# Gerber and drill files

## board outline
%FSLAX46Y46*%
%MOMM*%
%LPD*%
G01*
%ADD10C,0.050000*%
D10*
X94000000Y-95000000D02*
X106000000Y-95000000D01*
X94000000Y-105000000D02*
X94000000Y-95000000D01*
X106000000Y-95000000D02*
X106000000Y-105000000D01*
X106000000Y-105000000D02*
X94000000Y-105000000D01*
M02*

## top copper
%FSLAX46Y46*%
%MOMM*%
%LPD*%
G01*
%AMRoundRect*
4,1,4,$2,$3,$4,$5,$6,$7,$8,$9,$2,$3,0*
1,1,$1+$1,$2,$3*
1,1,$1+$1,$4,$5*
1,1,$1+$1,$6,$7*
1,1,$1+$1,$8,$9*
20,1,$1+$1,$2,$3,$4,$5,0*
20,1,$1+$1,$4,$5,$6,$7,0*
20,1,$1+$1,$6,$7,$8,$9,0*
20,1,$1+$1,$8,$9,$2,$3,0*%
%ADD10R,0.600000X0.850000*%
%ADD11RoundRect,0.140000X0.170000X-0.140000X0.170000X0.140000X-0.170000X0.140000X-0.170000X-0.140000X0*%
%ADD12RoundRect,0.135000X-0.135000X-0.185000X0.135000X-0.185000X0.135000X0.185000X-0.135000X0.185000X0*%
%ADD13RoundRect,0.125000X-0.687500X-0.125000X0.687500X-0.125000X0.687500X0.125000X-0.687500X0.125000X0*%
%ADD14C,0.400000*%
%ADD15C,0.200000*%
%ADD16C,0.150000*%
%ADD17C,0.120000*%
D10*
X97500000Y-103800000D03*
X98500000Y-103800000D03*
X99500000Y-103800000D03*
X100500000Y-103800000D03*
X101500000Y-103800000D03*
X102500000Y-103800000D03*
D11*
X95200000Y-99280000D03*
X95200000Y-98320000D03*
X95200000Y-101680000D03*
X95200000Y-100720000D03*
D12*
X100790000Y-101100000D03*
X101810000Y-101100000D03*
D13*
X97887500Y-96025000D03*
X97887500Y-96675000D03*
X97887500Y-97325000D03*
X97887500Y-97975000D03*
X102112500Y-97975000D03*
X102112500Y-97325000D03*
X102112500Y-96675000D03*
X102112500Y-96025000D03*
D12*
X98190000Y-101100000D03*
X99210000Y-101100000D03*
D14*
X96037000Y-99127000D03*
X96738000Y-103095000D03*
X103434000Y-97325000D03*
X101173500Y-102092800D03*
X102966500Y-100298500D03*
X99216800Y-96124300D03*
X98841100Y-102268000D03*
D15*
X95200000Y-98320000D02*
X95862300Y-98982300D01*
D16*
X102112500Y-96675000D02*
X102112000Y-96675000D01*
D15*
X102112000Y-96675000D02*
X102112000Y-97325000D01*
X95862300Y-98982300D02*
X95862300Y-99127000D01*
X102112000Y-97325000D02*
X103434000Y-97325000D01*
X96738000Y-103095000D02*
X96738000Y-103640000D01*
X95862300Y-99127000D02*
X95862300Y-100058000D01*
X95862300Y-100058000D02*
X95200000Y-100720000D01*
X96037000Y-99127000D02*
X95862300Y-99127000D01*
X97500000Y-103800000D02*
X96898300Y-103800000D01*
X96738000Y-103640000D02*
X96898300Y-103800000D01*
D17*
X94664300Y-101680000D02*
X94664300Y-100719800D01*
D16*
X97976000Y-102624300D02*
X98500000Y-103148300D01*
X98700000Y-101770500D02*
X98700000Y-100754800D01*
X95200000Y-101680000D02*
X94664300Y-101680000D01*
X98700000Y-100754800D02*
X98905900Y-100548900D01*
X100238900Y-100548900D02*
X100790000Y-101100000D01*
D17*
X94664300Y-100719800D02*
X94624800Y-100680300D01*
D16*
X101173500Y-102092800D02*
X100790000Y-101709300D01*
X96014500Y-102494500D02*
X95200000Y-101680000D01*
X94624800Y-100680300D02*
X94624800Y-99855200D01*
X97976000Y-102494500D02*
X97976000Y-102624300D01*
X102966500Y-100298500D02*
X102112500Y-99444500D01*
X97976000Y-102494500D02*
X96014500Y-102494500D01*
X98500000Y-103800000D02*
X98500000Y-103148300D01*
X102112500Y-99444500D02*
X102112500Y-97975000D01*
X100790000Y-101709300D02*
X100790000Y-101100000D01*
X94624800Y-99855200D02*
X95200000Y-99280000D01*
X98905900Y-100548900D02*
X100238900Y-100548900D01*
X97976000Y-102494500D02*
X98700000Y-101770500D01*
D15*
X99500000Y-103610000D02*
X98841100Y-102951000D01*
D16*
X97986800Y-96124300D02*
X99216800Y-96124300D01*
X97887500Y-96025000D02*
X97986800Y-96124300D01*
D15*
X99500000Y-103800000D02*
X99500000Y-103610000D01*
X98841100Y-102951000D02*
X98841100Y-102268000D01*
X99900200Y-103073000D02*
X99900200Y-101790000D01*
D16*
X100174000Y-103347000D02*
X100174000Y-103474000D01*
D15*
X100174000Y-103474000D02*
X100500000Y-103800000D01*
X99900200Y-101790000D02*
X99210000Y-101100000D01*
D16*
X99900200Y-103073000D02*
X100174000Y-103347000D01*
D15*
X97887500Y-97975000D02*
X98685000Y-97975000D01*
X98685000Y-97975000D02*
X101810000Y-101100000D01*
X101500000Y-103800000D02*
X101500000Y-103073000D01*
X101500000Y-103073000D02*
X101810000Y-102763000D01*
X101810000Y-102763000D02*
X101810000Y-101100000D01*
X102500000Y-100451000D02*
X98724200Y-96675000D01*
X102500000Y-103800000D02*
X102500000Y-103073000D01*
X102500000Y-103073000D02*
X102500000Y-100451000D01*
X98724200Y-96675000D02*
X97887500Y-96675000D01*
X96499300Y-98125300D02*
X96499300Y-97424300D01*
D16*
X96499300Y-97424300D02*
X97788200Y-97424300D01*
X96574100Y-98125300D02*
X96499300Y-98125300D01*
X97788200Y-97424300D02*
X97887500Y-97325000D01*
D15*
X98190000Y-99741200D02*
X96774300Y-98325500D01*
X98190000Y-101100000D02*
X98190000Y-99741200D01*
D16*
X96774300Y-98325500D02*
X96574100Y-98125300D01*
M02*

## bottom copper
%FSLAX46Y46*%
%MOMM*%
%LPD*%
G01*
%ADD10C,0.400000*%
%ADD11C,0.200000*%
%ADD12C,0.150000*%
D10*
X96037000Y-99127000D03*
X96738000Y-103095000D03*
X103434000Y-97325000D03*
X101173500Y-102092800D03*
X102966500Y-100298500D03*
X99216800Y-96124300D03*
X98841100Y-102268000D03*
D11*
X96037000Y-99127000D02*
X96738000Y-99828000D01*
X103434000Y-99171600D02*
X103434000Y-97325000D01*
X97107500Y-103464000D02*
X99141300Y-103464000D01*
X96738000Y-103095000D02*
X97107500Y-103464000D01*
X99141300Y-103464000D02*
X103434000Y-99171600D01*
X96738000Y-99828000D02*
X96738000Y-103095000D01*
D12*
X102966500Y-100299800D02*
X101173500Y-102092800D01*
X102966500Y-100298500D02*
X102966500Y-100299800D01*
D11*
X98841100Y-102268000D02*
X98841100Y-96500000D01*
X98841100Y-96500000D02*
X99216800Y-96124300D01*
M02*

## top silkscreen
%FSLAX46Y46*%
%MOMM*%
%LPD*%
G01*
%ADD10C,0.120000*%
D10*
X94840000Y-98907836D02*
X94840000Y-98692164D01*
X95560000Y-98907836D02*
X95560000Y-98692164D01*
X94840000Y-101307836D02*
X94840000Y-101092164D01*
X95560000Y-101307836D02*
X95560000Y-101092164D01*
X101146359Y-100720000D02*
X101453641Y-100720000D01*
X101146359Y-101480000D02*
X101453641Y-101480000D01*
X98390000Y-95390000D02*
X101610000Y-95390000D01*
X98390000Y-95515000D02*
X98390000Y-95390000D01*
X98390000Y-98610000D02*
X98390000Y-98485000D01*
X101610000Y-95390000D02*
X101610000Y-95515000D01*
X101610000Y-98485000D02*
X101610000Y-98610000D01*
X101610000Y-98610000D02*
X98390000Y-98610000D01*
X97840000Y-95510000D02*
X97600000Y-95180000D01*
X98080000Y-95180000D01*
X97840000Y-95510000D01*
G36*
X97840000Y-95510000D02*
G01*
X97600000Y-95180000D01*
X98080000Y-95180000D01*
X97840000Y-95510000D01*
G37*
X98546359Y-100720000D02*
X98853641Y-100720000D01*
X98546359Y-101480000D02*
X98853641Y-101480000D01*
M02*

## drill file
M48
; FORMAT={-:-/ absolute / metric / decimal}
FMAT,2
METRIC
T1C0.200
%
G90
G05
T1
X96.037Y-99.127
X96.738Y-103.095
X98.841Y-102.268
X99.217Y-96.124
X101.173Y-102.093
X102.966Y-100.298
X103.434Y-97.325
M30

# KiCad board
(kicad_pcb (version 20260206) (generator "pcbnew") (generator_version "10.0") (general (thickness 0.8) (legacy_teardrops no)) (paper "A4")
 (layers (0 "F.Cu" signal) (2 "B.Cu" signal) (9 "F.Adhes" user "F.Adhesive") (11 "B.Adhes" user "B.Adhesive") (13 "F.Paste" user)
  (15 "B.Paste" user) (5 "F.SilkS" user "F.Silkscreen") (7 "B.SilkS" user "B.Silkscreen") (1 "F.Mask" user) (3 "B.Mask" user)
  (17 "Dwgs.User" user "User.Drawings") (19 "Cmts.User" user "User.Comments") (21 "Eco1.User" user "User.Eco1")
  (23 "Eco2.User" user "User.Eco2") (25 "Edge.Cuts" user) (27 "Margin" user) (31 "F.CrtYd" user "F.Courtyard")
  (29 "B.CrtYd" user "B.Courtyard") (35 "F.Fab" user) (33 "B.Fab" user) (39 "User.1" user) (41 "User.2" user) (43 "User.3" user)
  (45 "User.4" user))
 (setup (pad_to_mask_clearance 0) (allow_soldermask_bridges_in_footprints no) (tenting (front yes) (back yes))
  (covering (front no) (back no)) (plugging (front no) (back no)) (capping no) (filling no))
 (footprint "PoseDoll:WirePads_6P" (layer "F.Cu") (at 100 103.8)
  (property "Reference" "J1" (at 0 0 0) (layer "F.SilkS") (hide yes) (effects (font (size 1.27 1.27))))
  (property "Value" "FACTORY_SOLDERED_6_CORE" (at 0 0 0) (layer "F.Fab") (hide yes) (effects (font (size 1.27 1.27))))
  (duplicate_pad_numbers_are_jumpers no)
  (pad "1" smd rect (at -2.5 0) (size 0.6 0.85) (layers "F.Cu" "F.Mask") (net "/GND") (thermal_bridge_angle 45))
  (pad "2" smd rect (at -1.5 0) (size 0.6 0.85) (layers "F.Cu" "F.Mask") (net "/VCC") (thermal_bridge_angle 45))
  (pad "3" smd rect (at -0.5 0) (size 0.6 0.85) (layers "F.Cu" "F.Mask") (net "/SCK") (thermal_bridge_angle 45))
  (pad "4" smd rect (at 0.5 0) (size 0.6 0.85) (layers "F.Cu" "F.Mask") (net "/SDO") (thermal_bridge_angle 45))
  (pad "5" smd rect (at 1.5 0) (size 0.6 0.85) (layers "F.Cu" "F.Mask") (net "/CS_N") (thermal_bridge_angle 45))
  (pad "6" smd rect (at 2.5 0) (size 0.6 0.85) (layers "F.Cu" "F.Mask") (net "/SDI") (thermal_bridge_angle 45)))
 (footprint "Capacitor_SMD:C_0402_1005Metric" (layer "F.Cu") (at 95.2 98.8 90)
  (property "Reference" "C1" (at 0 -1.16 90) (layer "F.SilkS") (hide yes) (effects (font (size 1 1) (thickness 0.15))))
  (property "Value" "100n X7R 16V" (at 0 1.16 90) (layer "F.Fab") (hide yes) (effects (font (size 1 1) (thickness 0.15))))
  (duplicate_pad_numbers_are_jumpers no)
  (fp_line (start -0.107836 -0.36) (end 0.107836 -0.36) (stroke (width 0.12) (type solid)) (layer "F.SilkS"))
  (fp_line (start -0.107836 0.36) (end 0.107836 0.36) (stroke (width 0.12) (type solid)) (layer "F.SilkS"))
  (pad "1" smd roundrect (at -0.48 0 90) (size 0.56 0.62) (layers "F.Cu" "F.Mask" "F.Paste") (roundrect_rratio 0.25) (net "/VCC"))
  (pad "2" smd roundrect (at 0.48 0 90) (size 0.56 0.62) (layers "F.Cu" "F.Mask" "F.Paste") (roundrect_rratio 0.25) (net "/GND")))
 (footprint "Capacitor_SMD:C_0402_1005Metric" (layer "F.Cu") (at 95.2 101.2 90)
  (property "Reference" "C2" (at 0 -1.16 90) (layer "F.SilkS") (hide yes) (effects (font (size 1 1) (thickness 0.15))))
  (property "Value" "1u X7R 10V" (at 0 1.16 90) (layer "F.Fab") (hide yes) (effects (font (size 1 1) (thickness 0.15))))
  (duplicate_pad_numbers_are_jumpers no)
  (fp_line (start -0.107836 -0.36) (end 0.107836 -0.36) (stroke (width 0.12) (type solid)) (layer "F.SilkS"))
  (fp_line (start -0.107836 0.36) (end 0.107836 0.36) (stroke (width 0.12) (type solid)) (layer "F.SilkS"))
  (pad "1" smd roundrect (at -0.48 0 90) (size 0.56 0.62) (layers "F.Cu" "F.Mask" "F.Paste") (roundrect_rratio 0.25) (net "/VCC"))
  (pad "2" smd roundrect (at 0.48 0 90) (size 0.56 0.62) (layers "F.Cu" "F.Mask" "F.Paste") (roundrect_rratio 0.25) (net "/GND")))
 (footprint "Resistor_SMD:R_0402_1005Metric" (layer "F.Cu") (at 101.3 101.1)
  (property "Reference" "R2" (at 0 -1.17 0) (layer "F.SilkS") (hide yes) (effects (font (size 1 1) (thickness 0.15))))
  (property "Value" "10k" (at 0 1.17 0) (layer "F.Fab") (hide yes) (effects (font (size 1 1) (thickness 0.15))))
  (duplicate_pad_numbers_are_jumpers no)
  (fp_line (start -0.153641 -0.38) (end 0.153641 -0.38) (stroke (width 0.12) (type solid)) (layer "F.SilkS"))
  (fp_line (start -0.153641 0.38) (end 0.153641 0.38) (stroke (width 0.12) (type solid)) (layer "F.SilkS"))
  (pad "1" smd roundrect (at -0.51 0) (size 0.54 0.64) (layers "F.Cu" "F.Mask" "F.Paste") (roundrect_rratio 0.25) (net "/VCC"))
  (pad "2" smd roundrect (at 0.51 0) (size 0.54 0.64) (layers "F.Cu" "F.Mask" "F.Paste") (roundrect_rratio 0.25) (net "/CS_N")))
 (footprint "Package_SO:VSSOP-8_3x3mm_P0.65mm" (layer "F.Cu") (at 100 97)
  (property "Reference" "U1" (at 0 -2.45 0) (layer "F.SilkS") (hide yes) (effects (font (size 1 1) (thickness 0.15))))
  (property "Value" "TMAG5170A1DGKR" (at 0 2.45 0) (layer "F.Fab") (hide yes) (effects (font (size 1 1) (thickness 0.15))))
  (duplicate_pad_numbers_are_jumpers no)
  (fp_line (start -1.61 -1.61) (end 1.61 -1.61) (stroke (width 0.12) (type solid)) (layer "F.SilkS"))
  (fp_line (start -1.61 -1.485) (end -1.61 -1.61) (stroke (width 0.12) (type solid)) (layer "F.SilkS"))
  (fp_line (start -1.61 1.61) (end -1.61 1.485) (stroke (width 0.12) (type solid)) (layer "F.SilkS"))
  (fp_line (start 1.61 -1.61) (end 1.61 -1.485) (stroke (width 0.12) (type solid)) (layer "F.SilkS"))
  (fp_line (start 1.61 1.485) (end 1.61 1.61) (stroke (width 0.12) (type solid)) (layer "F.SilkS"))
  (fp_line (start 1.61 1.61) (end -1.61 1.61) (stroke (width 0.12) (type solid)) (layer "F.SilkS"))
  (fp_poly (pts (xy -2.16 -1.49) (xy -2.4 -1.82) (xy -1.92 -1.82)) (stroke (width 0.12) (type solid)) (fill yes) (layer "F.SilkS"))
  (pad "1" smd roundrect (at -2.1125 -0.975) (size 1.625 0.5) (layers "F.Cu" "F.Mask" "F.Paste") (roundrect_rratio 0.25) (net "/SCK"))
  (pad "2" smd roundrect (at -2.1125 -0.325) (size 1.625 0.5) (layers "F.Cu" "F.Mask" "F.Paste") (roundrect_rratio 0.25) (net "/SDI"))
  (pad "3" smd roundrect (at -2.1125 0.325) (size 1.625 0.5) (layers "F.Cu" "F.Mask" "F.Paste") (roundrect_rratio 0.25) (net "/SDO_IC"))
  (pad "4" smd roundrect (at -2.1125 0.975) (size 1.625 0.5) (layers "F.Cu" "F.Mask" "F.Paste") (roundrect_rratio 0.25) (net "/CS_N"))
  (pad "5" smd roundrect (at 2.1125 0.975) (size 1.625 0.5) (layers "F.Cu" "F.Mask" "F.Paste") (roundrect_rratio 0.25) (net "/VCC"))
  (pad "6" smd roundrect (at 2.1125 0.325) (size 1.625 0.5) (layers "F.Cu" "F.Mask" "F.Paste") (roundrect_rratio 0.25) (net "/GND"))
  (pad "7" smd roundrect (at 2.1125 -0.325) (size 1.625 0.5) (layers "F.Cu" "F.Mask" "F.Paste") (roundrect_rratio 0.25) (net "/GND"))
  (pad "8" smd roundrect (at 2.1125 -0.975) (size 1.625 0.5) (layers "F.Cu" "F.Mask" "F.Paste") (roundrect_rratio 0.25)
   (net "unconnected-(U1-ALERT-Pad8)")))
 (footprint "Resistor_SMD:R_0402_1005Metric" (layer "F.Cu") (at 98.7 101.1)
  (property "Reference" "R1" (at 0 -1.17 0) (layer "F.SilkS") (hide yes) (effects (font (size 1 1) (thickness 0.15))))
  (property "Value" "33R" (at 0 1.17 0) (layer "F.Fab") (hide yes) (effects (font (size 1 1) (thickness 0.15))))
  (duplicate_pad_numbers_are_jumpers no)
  (fp_line (start -0.153641 -0.38) (end 0.153641 -0.38) (stroke (width 0.12) (type solid)) (layer "F.SilkS"))
  (fp_line (start -0.153641 0.38) (end 0.153641 0.38) (stroke (width 0.12) (type solid)) (layer "F.SilkS"))
  (pad "1" smd roundrect (at -0.51 0) (size 0.54 0.64) (layers "F.Cu" "F.Mask" "F.Paste") (roundrect_rratio 0.25) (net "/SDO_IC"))
  (pad "2" smd roundrect (at 0.51 0) (size 0.54 0.64) (layers "F.Cu" "F.Mask" "F.Paste") (roundrect_rratio 0.25) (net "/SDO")))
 (gr_line (start 94 95) (end 106 95) (stroke (width 0.05) (type default)) (layer "Edge.Cuts"))
 (gr_line (start 94 105) (end 94 95) (stroke (width 0.05) (type default)) (layer "Edge.Cuts"))
 (gr_line (start 106 95) (end 106 105) (stroke (width 0.05) (type default)) (layer "Edge.Cuts"))
 (gr_line (start 106 105) (end 94 105) (stroke (width 0.05) (type default)) (layer "Edge.Cuts"))
 (segment (start 95.2 98.32) (end 95.8623 98.9823) (width 0.2) (layer "F.Cu") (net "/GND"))
 (segment (start 102.1125 96.675) (end 102.112 96.675) (width 0.15) (layer "F.Cu") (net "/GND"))
 (segment (start 102.112 96.675) (end 102.112 97.325) (width 0.2) (layer "F.Cu") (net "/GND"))
 (segment (start 95.8623 98.9823) (end 95.8623 99.127) (width 0.2) (layer "F.Cu") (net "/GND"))
 (segment (start 102.112 97.325) (end 103.434 97.325) (width 0.2) (layer "F.Cu") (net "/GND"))
 (segment (start 96.738 103.095) (end 96.738 103.64) (width 0.2) (layer "F.Cu") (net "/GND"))
 (segment (start 95.8623 99.127) (end 95.8623 100.058) (width 0.2) (layer "F.Cu") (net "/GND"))
 (segment (start 95.8623 100.058) (end 95.2 100.72) (width 0.2) (layer "F.Cu") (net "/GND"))
 (segment (start 96.037 99.127) (end 95.8623 99.127) (width 0.2) (layer "F.Cu") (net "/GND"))
 (segment (start 97.5 103.8) (end 96.8983 103.8) (width 0.2) (layer "F.Cu") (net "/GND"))
 (segment (start 96.738 103.64) (end 96.8983 103.8) (width 0.2) (layer "F.Cu") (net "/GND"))
 (via (at 96.037 99.127) (size 0.4) (drill 0.2) (layers "F.Cu" "B.Cu") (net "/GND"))
 (via (at 96.738 103.095) (size 0.4) (drill 0.2) (layers "F.Cu" "B.Cu") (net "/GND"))
 (via (at 103.434 97.325) (size 0.4) (drill 0.2) (layers "F.Cu" "B.Cu") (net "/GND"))
 (segment (start 96.037 99.127) (end 96.738 99.828) (width 0.2) (layer "B.Cu") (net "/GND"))
 (segment (start 103.434 99.1716) (end 103.434 97.325) (width 0.2) (layer "B.Cu") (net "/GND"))
 (segment (start 97.1075 103.464) (end 99.1413 103.464) (width 0.2) (layer "B.Cu") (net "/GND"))
 (segment (start 96.738 103.095) (end 97.1075 103.464) (width 0.2) (layer "B.Cu") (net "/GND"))
 (segment (start 99.1413 103.464) (end 103.434 99.1716) (width 0.2) (layer "B.Cu") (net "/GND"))
 (segment (start 96.738 99.828) (end 96.738 103.095) (width 0.2) (layer "B.Cu") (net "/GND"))
 (segment (start 94.6643 101.68) (end 94.6643 100.7198) (width 0.12) (layer "F.Cu") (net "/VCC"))
 (segment (start 97.976 102.6243) (end 98.5 103.1483) (width 0.15) (layer "F.Cu") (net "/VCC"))
 (segment (start 98.7 101.7705) (end 98.7 100.7548) (width 0.15) (layer "F.Cu") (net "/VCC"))
 (segment (start 95.2 101.68) (end 94.6643 101.68) (width 0.15) (layer "F.Cu") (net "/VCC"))
 (segment (start 98.7 100.7548) (end 98.9059 100.5489) (width 0.15) (layer "F.Cu") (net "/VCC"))
 (segment (start 100.2389 100.5489) (end 100.79 101.1) (width 0.15) (layer "F.Cu") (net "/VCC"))
 (segment (start 94.6643 100.7198) (end 94.6248 100.6803) (width 0.12) (layer "F.Cu") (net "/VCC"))
 (segment (start 101.1735 102.0928) (end 100.79 101.7093) (width 0.15) (layer "F.Cu") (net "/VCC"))
 (segment (start 96.0145 102.4945) (end 95.2 101.68) (width 0.15) (layer "F.Cu") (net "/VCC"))
 (segment (start 94.6248 100.6803) (end 94.6248 99.8552) (width 0.15) (layer "F.Cu") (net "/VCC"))
 (segment (start 97.976 102.4945) (end 97.976 102.6243) (width 0.15) (layer "F.Cu") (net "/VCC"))
 (segment (start 102.9665 100.2985) (end 102.1125 99.4445) (width 0.15) (layer "F.Cu") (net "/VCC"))
 (segment (start 97.976 102.4945) (end 96.0145 102.4945) (width 0.15) (layer "F.Cu") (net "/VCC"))
 (segment (start 98.5 103.8) (end 98.5 103.1483) (width 0.15) (layer "F.Cu") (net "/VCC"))
 (segment (start 102.1125 99.4445) (end 102.1125 97.975) (width 0.15) (layer "F.Cu") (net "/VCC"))
 (segment (start 100.79 101.7093) (end 100.79 101.1) (width 0.15) (layer "F.Cu") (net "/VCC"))
 (segment (start 94.6248 99.8552) (end 95.2 99.28) (width 0.15) (layer "F.Cu") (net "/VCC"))
 (segment (start 98.9059 100.5489) (end 100.2389 100.5489) (width 0.15) (layer "F.Cu") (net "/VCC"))
 (segment (start 97.976 102.4945) (end 98.7 101.7705) (width 0.15) (layer "F.Cu") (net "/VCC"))
 (via (at 101.1735 102.0928) (size 0.4) (drill 0.2) (layers "F.Cu" "B.Cu") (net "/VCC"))
 (via (at 102.9665 100.2985) (size 0.4) (drill 0.2) (layers "F.Cu" "B.Cu") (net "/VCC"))
 (segment (start 102.9665 100.2998) (end 101.1735 102.0928) (width 0.15) (layer "B.Cu") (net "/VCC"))
 (segment (start 102.9665 100.2985) (end 102.9665 100.2998) (width 0.15) (layer "B.Cu") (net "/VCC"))
 (segment (start 99.5 103.61) (end 98.8411 102.951) (width 0.2) (layer "F.Cu") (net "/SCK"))
 (segment (start 97.9868 96.1243) (end 99.2168 96.1243) (width 0.15) (layer "F.Cu") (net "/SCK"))
 (segment (start 97.8875 96.025) (end 97.9868 96.1243) (width 0.15) (layer "F.Cu") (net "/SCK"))
 (segment (start 99.5 103.8) (end 99.5 103.61) (width 0.2) (layer "F.Cu") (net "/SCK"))
 (segment (start 98.8411 102.951) (end 98.8411 102.268) (width 0.2) (layer "F.Cu") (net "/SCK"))
 (via (at 99.2168 96.1243) (size 0.4) (drill 0.2) (layers "F.Cu" "B.Cu") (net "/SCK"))
 (via (at 98.8411 102.268) (size 0.4) (drill 0.2) (layers "F.Cu" "B.Cu") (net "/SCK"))
 (segment (start 98.8411 102.268) (end 98.8411 96.5) (width 0.2) (layer "B.Cu") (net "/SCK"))
 (segment (start 98.8411 96.5) (end 99.2168 96.1243) (width 0.2) (layer "B.Cu") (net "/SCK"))
 (segment (start 99.9002 103.073) (end 99.9002 101.79) (width 0.2) (layer "F.Cu") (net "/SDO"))
 (segment (start 100.174 103.347) (end 100.174 103.474) (width 0.15) (layer "F.Cu") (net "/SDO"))
 (segment (start 100.174 103.474) (end 100.5 103.8) (width 0.2) (layer "F.Cu") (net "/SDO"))
 (segment (start 99.9002 101.79) (end 99.21 101.1) (width 0.2) (layer "F.Cu") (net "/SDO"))
 (segment (start 99.9002 103.073) (end 100.174 103.347) (width 0.15) (layer "F.Cu") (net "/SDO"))
 (segment (start 97.8875 97.975) (end 98.685 97.975) (width 0.2) (layer "F.Cu") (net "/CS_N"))
 (segment (start 98.685 97.975) (end 101.81 101.1) (width 0.2) (layer "F.Cu") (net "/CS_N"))
 (segment (start 101.5 103.8) (end 101.5 103.073) (width 0.2) (layer "F.Cu") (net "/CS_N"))
 (segment (start 101.5 103.073) (end 101.81 102.763) (width 0.2) (layer "F.Cu") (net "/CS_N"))
 (segment (start 101.81 102.763) (end 101.81 101.1) (width 0.2) (layer "F.Cu") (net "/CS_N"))
 (segment (start 102.5 100.451) (end 98.7242 96.675) (width 0.2) (layer "F.Cu") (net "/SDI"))
 (segment (start 102.5 103.8) (end 102.5 103.073) (width 0.2) (layer "F.Cu") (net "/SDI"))
 (segment (start 102.5 103.073) (end 102.5 100.451) (width 0.2) (layer "F.Cu") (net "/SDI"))
 (segment (start 98.7242 96.675) (end 97.8875 96.675) (width 0.2) (layer "F.Cu") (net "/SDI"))
 (segment (start 96.4993 98.1253) (end 96.4993 97.4243) (width 0.2) (layer "F.Cu") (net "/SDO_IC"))
 (segment (start 96.4993 97.4243) (end 97.7882 97.4243) (width 0.15) (layer "F.Cu") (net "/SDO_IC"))
 (segment (start 96.5741 98.1253) (end 96.4993 98.1253) (width 0.15) (layer "F.Cu") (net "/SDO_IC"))
 (segment (start 97.7882 97.4243) (end 97.8875 97.325) (width 0.15) (layer "F.Cu") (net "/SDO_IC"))
 (segment (start 98.19 99.7412) (end 96.7743 98.3255) (width 0.2) (layer "F.Cu") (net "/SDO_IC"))
 (segment (start 98.19 101.1) (end 98.19 99.7412) (width 0.2) (layer "F.Cu") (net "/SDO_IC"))
 (segment (start 96.7743 98.3255) (end 96.5741 98.1253) (width 0.15) (layer "F.Cu") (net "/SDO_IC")))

